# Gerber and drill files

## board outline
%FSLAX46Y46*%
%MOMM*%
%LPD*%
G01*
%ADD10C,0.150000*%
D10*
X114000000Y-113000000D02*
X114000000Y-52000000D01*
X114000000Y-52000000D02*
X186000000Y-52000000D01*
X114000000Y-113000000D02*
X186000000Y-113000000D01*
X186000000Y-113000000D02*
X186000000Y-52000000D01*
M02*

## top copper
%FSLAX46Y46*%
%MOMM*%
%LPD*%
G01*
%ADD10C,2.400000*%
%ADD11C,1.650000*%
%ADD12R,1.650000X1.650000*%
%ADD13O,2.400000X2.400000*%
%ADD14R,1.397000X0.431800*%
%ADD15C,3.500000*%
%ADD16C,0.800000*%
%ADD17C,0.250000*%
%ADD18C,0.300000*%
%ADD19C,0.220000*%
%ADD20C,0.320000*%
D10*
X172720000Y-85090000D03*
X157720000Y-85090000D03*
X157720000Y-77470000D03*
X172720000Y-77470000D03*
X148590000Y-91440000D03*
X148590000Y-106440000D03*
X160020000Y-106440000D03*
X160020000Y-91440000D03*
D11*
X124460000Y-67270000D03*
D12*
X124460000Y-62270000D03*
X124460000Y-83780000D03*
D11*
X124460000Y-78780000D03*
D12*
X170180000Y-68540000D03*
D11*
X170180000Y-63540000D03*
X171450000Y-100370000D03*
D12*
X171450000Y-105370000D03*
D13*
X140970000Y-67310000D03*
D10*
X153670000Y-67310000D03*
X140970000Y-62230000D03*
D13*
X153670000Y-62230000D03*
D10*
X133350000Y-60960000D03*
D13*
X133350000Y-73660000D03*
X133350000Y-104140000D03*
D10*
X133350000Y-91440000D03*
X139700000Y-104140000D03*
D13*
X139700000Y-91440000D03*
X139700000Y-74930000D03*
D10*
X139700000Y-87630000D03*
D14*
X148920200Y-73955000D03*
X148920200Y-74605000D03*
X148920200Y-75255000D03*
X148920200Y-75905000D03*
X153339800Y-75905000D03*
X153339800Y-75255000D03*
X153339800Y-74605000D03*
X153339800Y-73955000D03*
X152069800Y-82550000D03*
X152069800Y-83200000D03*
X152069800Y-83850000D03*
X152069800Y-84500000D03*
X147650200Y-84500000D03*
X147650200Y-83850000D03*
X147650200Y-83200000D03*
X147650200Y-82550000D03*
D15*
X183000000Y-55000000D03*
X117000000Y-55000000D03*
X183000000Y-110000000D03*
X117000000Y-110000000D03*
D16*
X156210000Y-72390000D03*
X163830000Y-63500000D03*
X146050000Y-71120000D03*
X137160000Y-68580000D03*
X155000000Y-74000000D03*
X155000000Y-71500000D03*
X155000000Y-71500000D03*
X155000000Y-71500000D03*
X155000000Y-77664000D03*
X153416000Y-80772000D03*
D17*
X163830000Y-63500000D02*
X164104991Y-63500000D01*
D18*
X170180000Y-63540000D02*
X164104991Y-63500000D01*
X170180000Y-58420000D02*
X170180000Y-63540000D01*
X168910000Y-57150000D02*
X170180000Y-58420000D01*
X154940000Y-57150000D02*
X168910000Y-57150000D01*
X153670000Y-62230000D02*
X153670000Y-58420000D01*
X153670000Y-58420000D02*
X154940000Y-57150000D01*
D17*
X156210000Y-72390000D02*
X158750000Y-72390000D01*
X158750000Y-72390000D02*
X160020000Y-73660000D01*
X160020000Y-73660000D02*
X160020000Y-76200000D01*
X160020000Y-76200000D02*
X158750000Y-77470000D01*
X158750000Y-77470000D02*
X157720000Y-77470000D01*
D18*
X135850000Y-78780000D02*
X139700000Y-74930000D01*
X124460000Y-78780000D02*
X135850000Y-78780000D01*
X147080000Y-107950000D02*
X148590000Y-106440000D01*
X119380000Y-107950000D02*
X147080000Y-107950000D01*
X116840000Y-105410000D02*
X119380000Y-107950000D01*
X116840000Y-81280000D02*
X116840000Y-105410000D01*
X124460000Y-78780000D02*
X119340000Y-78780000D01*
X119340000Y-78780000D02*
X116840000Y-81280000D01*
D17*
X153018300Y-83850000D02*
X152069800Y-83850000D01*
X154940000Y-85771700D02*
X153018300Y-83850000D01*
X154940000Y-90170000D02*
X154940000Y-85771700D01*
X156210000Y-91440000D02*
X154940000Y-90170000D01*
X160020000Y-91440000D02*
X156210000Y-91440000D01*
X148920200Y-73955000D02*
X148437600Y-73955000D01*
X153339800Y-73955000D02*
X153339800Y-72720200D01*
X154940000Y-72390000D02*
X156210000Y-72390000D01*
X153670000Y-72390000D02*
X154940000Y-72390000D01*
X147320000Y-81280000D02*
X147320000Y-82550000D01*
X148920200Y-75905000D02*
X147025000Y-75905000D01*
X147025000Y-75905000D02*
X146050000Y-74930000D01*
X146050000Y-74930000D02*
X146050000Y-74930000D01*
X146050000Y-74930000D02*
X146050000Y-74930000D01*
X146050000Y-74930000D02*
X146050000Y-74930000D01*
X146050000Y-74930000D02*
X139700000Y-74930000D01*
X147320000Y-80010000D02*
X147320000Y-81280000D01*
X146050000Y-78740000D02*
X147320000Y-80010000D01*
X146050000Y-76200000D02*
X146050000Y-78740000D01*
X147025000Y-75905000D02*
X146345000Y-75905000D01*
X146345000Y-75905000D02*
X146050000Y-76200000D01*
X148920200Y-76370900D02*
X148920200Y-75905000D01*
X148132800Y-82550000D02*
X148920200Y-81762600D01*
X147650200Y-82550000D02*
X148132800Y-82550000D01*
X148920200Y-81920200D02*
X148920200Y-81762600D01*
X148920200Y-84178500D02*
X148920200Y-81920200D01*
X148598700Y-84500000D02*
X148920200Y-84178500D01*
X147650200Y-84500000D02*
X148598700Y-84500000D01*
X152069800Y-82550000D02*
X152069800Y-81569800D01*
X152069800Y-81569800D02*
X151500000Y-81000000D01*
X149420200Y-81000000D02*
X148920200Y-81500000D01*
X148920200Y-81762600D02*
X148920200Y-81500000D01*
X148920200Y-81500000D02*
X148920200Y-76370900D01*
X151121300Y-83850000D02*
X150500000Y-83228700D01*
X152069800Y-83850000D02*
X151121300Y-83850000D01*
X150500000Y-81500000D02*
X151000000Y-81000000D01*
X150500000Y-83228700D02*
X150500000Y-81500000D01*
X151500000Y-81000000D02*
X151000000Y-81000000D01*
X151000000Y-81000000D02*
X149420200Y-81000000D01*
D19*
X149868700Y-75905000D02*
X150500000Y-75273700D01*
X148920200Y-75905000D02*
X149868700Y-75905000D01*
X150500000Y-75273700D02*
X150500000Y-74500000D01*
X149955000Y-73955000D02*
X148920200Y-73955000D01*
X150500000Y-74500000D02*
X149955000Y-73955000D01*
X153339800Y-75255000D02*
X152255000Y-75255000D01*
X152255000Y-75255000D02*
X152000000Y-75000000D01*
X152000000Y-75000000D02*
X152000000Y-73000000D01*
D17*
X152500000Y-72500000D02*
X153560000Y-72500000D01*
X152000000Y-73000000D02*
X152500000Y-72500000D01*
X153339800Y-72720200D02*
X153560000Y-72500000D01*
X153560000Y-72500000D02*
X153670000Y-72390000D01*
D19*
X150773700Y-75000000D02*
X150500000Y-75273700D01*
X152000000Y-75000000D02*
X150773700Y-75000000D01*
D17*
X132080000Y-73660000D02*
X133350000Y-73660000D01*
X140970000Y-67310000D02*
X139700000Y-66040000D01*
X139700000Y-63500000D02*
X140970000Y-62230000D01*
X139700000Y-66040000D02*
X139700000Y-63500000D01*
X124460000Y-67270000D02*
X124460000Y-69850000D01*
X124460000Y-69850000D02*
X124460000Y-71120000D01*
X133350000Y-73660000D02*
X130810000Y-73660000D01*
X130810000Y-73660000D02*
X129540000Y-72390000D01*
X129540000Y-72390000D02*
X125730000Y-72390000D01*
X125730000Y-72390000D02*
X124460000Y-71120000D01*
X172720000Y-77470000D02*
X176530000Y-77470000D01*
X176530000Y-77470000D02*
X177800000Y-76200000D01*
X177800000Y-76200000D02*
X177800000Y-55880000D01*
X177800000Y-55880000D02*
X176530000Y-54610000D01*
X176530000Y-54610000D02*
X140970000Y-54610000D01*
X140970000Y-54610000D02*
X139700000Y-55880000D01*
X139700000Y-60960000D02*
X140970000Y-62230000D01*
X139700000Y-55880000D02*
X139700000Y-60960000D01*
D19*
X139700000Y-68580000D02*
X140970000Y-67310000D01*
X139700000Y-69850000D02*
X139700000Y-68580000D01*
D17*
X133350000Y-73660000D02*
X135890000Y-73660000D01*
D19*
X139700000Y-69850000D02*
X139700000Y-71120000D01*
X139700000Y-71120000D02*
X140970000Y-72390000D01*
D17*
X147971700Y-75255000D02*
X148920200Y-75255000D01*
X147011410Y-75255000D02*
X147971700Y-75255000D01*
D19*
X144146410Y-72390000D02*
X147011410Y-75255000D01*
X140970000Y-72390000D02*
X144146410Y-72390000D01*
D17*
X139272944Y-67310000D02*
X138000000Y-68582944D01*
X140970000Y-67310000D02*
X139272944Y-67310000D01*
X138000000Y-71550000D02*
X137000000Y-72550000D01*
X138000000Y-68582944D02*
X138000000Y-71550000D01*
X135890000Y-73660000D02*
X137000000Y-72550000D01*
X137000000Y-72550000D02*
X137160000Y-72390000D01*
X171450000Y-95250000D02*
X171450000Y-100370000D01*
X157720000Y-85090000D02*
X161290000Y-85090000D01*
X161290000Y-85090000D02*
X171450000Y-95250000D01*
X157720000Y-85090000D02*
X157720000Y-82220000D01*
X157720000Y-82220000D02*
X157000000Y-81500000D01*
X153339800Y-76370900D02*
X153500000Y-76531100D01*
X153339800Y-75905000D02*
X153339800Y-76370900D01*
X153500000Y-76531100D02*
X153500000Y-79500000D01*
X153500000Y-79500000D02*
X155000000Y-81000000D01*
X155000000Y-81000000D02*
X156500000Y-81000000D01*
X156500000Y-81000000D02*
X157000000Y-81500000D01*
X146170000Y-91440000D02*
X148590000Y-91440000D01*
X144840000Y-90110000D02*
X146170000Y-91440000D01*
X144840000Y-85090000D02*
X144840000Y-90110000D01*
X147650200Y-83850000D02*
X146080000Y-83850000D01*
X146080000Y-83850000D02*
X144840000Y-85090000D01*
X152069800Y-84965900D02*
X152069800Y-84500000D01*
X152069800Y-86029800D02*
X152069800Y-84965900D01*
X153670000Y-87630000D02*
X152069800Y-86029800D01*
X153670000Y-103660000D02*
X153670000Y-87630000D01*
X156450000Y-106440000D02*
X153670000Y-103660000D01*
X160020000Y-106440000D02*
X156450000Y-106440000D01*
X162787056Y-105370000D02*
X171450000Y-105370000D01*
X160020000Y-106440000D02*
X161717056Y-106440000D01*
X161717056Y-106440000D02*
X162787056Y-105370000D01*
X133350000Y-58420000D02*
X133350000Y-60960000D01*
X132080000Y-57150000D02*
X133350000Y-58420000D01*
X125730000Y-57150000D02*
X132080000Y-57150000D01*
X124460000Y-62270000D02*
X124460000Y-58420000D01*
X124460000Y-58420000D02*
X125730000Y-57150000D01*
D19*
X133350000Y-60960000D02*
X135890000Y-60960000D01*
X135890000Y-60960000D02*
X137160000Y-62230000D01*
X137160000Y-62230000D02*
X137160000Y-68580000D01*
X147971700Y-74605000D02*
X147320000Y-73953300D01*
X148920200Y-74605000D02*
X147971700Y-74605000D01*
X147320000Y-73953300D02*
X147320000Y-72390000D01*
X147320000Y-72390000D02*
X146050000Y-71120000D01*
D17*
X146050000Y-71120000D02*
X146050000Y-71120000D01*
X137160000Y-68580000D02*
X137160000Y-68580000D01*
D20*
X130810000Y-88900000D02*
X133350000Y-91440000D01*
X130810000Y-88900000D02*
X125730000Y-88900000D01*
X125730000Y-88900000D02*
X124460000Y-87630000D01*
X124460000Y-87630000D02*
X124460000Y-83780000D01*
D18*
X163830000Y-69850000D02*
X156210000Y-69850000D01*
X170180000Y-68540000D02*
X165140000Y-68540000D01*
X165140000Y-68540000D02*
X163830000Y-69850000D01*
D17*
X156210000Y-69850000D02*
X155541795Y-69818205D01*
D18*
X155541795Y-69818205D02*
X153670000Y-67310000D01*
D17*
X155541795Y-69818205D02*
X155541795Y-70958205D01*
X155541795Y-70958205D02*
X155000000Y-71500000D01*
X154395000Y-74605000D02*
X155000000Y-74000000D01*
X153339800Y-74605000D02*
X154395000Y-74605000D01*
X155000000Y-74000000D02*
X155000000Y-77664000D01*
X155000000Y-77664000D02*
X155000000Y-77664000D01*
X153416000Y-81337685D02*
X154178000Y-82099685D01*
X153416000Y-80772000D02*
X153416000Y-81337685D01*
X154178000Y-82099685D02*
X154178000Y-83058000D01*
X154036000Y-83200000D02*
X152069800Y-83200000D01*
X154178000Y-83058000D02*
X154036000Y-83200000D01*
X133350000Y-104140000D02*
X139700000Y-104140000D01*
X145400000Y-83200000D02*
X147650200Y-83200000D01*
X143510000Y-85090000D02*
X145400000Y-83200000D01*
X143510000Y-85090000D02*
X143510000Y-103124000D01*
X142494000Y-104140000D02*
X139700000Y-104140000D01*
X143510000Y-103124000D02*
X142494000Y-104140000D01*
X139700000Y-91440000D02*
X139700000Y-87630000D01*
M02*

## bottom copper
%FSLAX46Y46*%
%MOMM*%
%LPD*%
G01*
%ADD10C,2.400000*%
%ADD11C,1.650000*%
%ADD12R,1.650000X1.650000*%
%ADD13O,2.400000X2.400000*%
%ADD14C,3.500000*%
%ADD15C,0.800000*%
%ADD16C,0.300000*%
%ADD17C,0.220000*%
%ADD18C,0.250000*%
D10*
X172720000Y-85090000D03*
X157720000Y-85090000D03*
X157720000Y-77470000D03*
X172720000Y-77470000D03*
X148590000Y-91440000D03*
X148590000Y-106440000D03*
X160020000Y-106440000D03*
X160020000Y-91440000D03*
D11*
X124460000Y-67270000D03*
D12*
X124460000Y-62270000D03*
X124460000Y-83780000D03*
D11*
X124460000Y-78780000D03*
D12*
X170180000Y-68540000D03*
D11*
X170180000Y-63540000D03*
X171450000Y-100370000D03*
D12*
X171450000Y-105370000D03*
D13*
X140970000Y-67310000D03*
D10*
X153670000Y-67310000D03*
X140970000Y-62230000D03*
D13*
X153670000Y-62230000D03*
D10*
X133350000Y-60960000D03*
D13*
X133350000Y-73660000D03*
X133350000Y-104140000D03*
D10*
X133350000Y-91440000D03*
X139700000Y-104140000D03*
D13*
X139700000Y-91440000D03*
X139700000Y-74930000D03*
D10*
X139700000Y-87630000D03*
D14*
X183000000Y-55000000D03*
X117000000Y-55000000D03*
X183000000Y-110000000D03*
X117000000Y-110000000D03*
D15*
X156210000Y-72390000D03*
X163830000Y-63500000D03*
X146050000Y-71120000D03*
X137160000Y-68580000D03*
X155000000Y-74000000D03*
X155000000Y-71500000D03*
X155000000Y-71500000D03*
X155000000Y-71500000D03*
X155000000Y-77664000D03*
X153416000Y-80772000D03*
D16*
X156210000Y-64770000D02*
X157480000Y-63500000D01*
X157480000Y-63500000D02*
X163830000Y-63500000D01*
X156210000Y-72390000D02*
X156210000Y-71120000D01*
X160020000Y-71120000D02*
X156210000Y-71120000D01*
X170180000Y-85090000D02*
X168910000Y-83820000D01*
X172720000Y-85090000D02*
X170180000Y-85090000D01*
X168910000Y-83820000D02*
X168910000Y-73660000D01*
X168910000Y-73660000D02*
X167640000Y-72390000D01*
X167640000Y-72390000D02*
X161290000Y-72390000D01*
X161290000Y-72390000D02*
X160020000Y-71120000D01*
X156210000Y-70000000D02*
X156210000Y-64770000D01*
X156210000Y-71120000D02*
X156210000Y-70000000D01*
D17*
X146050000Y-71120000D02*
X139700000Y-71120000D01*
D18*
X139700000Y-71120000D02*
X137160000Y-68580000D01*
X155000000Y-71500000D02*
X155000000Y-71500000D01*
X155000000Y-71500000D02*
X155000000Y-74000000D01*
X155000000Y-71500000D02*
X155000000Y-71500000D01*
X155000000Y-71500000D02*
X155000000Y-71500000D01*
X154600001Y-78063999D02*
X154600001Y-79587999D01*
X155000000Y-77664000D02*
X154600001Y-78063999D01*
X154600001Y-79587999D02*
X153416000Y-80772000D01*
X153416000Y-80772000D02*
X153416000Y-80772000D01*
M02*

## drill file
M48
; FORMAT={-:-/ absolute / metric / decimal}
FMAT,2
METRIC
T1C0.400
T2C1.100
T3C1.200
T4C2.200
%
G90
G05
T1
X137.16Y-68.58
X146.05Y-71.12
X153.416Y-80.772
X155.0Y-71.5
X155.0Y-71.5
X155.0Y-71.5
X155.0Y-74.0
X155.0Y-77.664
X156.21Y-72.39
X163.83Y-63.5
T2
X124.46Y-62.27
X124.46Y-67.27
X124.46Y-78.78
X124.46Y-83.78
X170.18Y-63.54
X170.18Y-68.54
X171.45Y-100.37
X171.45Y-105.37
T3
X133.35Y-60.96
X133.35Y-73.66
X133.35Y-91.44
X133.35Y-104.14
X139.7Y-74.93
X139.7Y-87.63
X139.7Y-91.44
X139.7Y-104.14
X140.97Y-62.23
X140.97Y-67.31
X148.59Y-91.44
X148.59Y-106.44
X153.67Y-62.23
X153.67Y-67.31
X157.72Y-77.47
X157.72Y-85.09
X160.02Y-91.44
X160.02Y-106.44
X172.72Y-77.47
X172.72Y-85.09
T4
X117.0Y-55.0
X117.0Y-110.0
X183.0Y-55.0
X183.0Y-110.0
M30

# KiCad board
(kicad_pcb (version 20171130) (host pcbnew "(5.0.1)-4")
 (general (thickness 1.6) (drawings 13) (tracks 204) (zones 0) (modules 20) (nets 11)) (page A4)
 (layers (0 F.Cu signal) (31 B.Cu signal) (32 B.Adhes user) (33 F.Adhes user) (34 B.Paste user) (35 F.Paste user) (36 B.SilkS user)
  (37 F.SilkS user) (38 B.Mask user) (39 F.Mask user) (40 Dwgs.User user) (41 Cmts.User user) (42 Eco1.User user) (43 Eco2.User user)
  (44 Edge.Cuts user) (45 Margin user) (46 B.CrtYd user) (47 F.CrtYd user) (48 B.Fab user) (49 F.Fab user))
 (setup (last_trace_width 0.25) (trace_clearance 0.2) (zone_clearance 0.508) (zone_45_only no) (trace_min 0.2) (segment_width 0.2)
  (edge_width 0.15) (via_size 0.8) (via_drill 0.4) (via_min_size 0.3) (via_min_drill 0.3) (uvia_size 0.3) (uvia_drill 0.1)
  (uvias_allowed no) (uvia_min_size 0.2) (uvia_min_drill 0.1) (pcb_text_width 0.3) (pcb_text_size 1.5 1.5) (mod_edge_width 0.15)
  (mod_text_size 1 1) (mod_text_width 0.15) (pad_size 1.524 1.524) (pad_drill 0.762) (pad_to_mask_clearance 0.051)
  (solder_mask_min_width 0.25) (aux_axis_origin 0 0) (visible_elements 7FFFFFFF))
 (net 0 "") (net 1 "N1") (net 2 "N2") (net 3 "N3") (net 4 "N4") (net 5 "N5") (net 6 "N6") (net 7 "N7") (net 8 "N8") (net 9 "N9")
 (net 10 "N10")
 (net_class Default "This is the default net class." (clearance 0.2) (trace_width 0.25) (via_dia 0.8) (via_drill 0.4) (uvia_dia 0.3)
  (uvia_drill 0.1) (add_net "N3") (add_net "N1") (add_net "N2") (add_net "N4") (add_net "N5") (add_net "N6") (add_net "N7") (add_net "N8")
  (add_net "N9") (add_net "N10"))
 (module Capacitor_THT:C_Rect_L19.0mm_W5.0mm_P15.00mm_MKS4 (layer F.Cu) (at 172.72 85.09 180)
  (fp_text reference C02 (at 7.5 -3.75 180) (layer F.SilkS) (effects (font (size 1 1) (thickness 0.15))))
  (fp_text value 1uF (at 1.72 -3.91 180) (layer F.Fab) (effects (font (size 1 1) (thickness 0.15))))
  (pad 1 thru_hole circle (at 0 0 180) (size 2.4 2.4) (drill 1.2) (layers *.Cu *.Mask) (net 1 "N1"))
  (pad 2 thru_hole circle (at 15 0 180) (size 2.4 2.4) (drill 1.2) (layers *.Cu *.Mask) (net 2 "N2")))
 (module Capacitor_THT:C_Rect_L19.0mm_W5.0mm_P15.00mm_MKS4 (layer F.Cu) (at 172.72 77.47 180)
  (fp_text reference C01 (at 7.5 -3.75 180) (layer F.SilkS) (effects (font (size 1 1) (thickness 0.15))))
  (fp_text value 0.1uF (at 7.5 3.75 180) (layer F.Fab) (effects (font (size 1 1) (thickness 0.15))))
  (pad 2 thru_hole circle (at 15 0 180) (size 2.4 2.4) (drill 1.2) (layers *.Cu *.Mask) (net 1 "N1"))
  (pad 1 thru_hole circle (at 0 0 180) (size 2.4 2.4) (drill 1.2) (layers *.Cu *.Mask) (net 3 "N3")))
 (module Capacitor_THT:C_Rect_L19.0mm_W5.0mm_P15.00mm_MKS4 (layer F.Cu) (at 148.59 91.44 270)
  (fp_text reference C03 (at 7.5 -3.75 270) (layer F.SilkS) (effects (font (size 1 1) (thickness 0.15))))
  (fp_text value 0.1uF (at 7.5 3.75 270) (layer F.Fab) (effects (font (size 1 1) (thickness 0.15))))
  (pad 1 thru_hole circle (at 0 0 270) (size 2.4 2.4) (drill 1.2) (layers *.Cu *.Mask) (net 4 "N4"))
  (pad 2 thru_hole circle (at 15 0 270) (size 2.4 2.4) (drill 1.2) (layers *.Cu *.Mask) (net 1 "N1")))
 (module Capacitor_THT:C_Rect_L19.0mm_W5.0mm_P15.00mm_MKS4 (layer F.Cu) (at 160.02 91.44 270)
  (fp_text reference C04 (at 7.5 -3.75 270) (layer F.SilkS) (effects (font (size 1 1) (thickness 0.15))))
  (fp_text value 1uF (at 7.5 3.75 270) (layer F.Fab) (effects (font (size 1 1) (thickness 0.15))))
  (pad 2 thru_hole circle (at 15 0 270) (size 2.4 2.4) (drill 1.2) (layers *.Cu *.Mask) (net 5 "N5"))
  (pad 1 thru_hole circle (at 0 0 270) (size 2.4 2.4) (drill 1.2) (layers *.Cu *.Mask) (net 1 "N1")))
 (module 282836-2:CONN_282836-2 (layer F.Cu) (at 124.46 64.77 270)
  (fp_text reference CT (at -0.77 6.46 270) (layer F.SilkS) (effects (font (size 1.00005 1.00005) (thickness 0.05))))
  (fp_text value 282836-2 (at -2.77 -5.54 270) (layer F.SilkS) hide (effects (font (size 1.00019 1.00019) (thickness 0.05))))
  (pad 2 thru_hole circle (at 2.5 0 270) (size 1.65 1.65) (drill 1.1) (layers *.Cu *.Mask) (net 3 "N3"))
  (pad 1 thru_hole rect (at -2.5 0 270) (size 1.65 1.65) (drill 1.1) (layers *.Cu *.Mask) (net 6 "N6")))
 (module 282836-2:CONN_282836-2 (layer F.Cu) (at 124.46 81.28 90)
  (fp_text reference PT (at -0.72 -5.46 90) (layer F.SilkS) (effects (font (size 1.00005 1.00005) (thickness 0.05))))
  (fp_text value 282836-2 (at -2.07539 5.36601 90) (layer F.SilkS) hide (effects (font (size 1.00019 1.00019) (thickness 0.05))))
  (pad 1 thru_hole rect (at -2.5 0 90) (size 1.65 1.65) (drill 1.1) (layers *.Cu *.Mask) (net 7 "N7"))
  (pad 2 thru_hole circle (at 2.5 0 90) (size 1.65 1.65) (drill 1.1) (layers *.Cu *.Mask) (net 1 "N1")))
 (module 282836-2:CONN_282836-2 (layer F.Cu) (at 170.18 66.04 90)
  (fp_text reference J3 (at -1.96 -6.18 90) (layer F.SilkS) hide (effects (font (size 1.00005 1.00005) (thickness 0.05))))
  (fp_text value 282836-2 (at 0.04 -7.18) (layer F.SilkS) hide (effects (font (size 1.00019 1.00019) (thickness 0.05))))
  (pad 1 thru_hole rect (at -2.5 0 90) (size 1.65 1.65) (drill 1.1) (layers *.Cu *.Mask) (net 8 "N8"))
  (pad 2 thru_hole circle (at 2.5 0 90) (size 1.65 1.65) (drill 1.1) (layers *.Cu *.Mask) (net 1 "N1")))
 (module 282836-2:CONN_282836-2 (layer F.Cu) (at 171.45 102.87 90)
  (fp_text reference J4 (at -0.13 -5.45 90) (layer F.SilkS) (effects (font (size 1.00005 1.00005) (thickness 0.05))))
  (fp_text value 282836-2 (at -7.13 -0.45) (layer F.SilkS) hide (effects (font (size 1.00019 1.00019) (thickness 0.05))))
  (pad 2 thru_hole circle (at 2.5 0 90) (size 1.65 1.65) (drill 1.1) (layers *.Cu *.Mask) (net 2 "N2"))
  (pad 1 thru_hole rect (at -2.5 0 90) (size 1.65 1.65) (drill 1.1) (layers *.Cu *.Mask) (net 5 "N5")))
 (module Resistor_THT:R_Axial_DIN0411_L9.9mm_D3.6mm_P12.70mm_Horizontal (layer F.Cu) (at 153.67 67.31 180)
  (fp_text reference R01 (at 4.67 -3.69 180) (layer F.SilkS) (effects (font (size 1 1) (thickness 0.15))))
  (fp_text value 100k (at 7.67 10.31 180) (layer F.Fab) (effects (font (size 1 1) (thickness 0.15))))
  (pad 2 thru_hole oval (at 12.7 0 180) (size 2.4 2.4) (drill 1.2) (layers *.Cu *.Mask) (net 3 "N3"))
  (pad 1 thru_hole circle (at 0 0 180) (size 2.4 2.4) (drill 1.2) (layers *.Cu *.Mask) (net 8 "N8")))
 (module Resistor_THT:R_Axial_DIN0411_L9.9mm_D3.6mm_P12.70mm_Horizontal (layer F.Cu) (at 140.97 62.23)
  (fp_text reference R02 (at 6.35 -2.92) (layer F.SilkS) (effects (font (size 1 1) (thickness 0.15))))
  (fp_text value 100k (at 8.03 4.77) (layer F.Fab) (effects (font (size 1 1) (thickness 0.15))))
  (pad 1 thru_hole circle (at 0 0) (size 2.4 2.4) (drill 1.2) (layers *.Cu *.Mask) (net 3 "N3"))
  (pad 2 thru_hole oval (at 12.7 0) (size 2.4 2.4) (drill 1.2) (layers *.Cu *.Mask) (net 1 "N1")))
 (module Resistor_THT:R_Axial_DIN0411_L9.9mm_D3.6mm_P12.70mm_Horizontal (layer F.Cu) (at 133.35 60.96 270)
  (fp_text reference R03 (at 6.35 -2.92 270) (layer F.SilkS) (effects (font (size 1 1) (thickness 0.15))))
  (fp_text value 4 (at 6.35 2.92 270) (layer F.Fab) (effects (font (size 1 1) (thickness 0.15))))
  (pad 1 thru_hole circle (at 0 0 270) (size 2.4 2.4) (drill 1.2) (layers *.Cu *.Mask) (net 6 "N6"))
  (pad 2 thru_hole oval (at 12.7 0 270) (size 2.4 2.4) (drill 1.2) (layers *.Cu *.Mask) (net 3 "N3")))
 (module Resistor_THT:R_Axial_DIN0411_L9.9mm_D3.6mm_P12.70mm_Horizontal (layer F.Cu) (at 133.35 91.44 270)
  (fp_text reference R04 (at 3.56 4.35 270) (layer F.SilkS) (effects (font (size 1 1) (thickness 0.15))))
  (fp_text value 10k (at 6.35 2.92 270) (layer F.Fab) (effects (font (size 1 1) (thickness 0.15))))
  (pad 2 thru_hole oval (at 12.7 0 270) (size 2.4 2.4) (drill 1.2) (layers *.Cu *.Mask) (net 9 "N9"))
  (pad 1 thru_hole circle (at 0 0 270) (size 2.4 2.4) (drill 1.2) (layers *.Cu *.Mask) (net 7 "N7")))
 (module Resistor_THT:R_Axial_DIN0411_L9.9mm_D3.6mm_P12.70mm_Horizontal (layer F.Cu) (at 139.7 104.14 90)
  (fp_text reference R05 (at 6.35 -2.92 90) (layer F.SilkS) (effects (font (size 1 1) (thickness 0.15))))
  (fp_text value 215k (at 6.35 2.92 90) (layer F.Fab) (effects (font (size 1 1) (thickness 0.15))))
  (pad 1 thru_hole circle (at 0 0 90) (size 2.4 2.4) (drill 1.2) (layers *.Cu *.Mask) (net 9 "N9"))
  (pad 2 thru_hole oval (at 12.7 0 90) (size 2.4 2.4) (drill 1.2) (layers *.Cu *.Mask) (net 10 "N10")))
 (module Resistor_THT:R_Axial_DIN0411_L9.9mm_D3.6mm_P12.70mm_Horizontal (layer F.Cu) (at 139.7 87.63 90)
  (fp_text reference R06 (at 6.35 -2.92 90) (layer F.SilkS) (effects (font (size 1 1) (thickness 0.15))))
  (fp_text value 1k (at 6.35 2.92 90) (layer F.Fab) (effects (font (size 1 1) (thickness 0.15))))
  (pad 2 thru_hole oval (at 12.7 0 90) (size 2.4 2.4) (drill 1.2) (layers *.Cu *.Mask) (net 1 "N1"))
  (pad 1 thru_hole circle (at 0 0 90) (size 2.4 2.4) (drill 1.2) (layers *.Cu *.Mask) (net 10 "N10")))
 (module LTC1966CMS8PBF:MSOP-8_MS (layer F.Cu) (at 151.13 74.93)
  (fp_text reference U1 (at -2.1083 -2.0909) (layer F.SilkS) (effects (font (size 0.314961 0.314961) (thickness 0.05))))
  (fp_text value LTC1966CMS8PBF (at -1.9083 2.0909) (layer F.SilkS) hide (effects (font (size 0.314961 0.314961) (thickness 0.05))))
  (pad 1 smd rect (at -2.2098 -0.975) (size 1.397 0.4318) (layers F.Cu F.Paste F.Mask) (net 1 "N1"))
  (pad 2 smd rect (at -2.2098 -0.325) (size 1.397 0.4318) (layers F.Cu F.Paste F.Mask) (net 6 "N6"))
  (pad 3 smd rect (at -2.2098 0.325) (size 1.397 0.4318) (layers F.Cu F.Paste F.Mask) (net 3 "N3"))
  (pad 4 smd rect (at -2.2098 0.975) (size 1.397 0.4318) (layers F.Cu F.Paste F.Mask) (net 1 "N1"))
  (pad 5 smd rect (at 2.2098 0.975) (size 1.397 0.4318) (layers F.Cu F.Paste F.Mask) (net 2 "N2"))
  (pad 6 smd rect (at 2.2098 0.325) (size 1.397 0.4318) (layers F.Cu F.Paste F.Mask) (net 1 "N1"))
  (pad 7 smd rect (at 2.2098 -0.325) (size 1.397 0.4318) (layers F.Cu F.Paste F.Mask) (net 8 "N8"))
  (pad 8 smd rect (at 2.2098 -0.975) (size 1.397 0.4318) (layers F.Cu F.Paste F.Mask) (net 1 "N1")))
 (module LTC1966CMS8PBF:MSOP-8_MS (layer F.Cu) (at 149.86 83.525)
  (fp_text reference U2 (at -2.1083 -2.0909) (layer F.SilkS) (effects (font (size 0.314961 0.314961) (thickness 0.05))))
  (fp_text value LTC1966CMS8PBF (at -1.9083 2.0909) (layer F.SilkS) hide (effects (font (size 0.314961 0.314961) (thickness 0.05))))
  (pad 8 smd rect (at 2.2098 -0.975) (size 1.397 0.4318) (layers F.Cu F.Paste F.Mask) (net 1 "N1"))
  (pad 7 smd rect (at 2.2098 -0.325) (size 1.397 0.4318) (layers F.Cu F.Paste F.Mask) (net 8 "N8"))
  (pad 6 smd rect (at 2.2098 0.325) (size 1.397 0.4318) (layers F.Cu F.Paste F.Mask) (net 1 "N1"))
  (pad 5 smd rect (at 2.2098 0.975) (size 1.397 0.4318) (layers F.Cu F.Paste F.Mask) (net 5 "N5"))
  (pad 4 smd rect (at -2.2098 0.975) (size 1.397 0.4318) (layers F.Cu F.Paste F.Mask) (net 1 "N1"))
  (pad 3 smd rect (at -2.2098 0.325) (size 1.397 0.4318) (layers F.Cu F.Paste F.Mask) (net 4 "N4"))
  (pad 2 smd rect (at -2.2098 -0.325) (size 1.397 0.4318) (layers F.Cu F.Paste F.Mask) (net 9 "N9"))
  (pad 1 smd rect (at -2.2098 -0.975) (size 1.397 0.4318) (layers F.Cu F.Paste F.Mask) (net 1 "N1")))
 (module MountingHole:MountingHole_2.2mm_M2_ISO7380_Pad (layer F.Cu) (at 183 55)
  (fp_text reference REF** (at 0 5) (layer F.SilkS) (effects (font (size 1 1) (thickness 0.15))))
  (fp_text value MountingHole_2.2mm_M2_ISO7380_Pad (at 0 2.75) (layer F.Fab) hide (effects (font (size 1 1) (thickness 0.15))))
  (pad 1 thru_hole circle (at 0 0) (size 3.5 3.5) (drill 2.2) (layers *.Cu *.Mask)))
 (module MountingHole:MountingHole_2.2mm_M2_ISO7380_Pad (layer F.Cu) (at 117 55)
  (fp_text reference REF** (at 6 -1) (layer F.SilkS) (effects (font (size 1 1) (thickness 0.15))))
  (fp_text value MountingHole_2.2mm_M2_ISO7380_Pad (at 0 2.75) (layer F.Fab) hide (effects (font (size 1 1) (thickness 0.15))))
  (pad 1 thru_hole circle (at 0 0) (size 3.5 3.5) (drill 2.2) (layers *.Cu *.Mask)))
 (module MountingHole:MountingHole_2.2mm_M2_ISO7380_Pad (layer F.Cu) (at 183 110)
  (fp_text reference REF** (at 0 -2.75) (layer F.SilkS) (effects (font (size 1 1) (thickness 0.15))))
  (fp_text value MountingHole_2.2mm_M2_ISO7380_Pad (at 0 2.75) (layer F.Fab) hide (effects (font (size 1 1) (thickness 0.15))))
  (pad 1 thru_hole circle (at 0 0) (size 3.5 3.5) (drill 2.2) (layers *.Cu *.Mask)))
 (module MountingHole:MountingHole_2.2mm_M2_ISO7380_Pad (layer F.Cu) (at 117 110)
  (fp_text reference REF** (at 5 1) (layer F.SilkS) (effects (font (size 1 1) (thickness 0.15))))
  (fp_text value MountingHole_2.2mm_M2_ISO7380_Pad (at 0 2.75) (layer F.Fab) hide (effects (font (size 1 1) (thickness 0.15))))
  (pad 1 thru_hole circle (at 0 0) (size 3.5 3.5) (drill 2.2) (layers *.Cu *.Mask)))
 (gr_line (start 114 113) (end 114 52) (layer Edge.Cuts) (width 0.15))
 (gr_line (start 114 52) (end 186 52) (layer Edge.Cuts) (width 0.15))
 (gr_line (start 114 113) (end 186 113) (layer Edge.Cuts) (width 0.15))
 (gr_line (start 186 113) (end 186 52) (layer Edge.Cuts) (width 0.15))
 (via (at 156.21 72.39) (size 0.8) (drill 0.4) (layers F.Cu B.Cu) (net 1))
 (via (at 163.83 63.5) (size 0.8) (drill 0.4) (layers F.Cu B.Cu) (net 1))
 (segment (start 163.83 63.5) (end 164.104991 63.5) (width 0.25) (layer F.Cu) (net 1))
 (segment (start 170.18 63.54) (end 164.104991 63.5) (width 0.3) (layer F.Cu) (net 1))
 (segment (start 170.18 58.42) (end 170.18 63.54) (width 0.3) (layer F.Cu) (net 1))
 (segment (start 168.91 57.15) (end 170.18 58.42) (width 0.3) (layer F.Cu) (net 1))
 (segment (start 154.94 57.15) (end 168.91 57.15) (width 0.3) (layer F.Cu) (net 1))
 (segment (start 153.67 62.23) (end 153.67 58.42) (width 0.3) (layer F.Cu) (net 1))
 (segment (start 153.67 58.42) (end 154.94 57.15) (width 0.3) (layer F.Cu) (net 1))
 (segment (start 156.21 64.77) (end 157.48 63.5) (width 0.3) (layer B.Cu) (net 1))
 (segment (start 157.48 63.5) (end 163.83 63.5) (width 0.3) (layer B.Cu) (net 1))
 (segment (start 156.21 72.39) (end 158.75 72.39) (width 0.25) (layer F.Cu) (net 1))
 (segment (start 158.75 72.39) (end 160.02 73.66) (width 0.25) (layer F.Cu) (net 1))
 (segment (start 160.02 73.66) (end 160.02 76.2) (width 0.25) (layer F.Cu) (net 1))
 (segment (start 160.02 76.2) (end 158.75 77.47) (width 0.25) (layer F.Cu) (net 1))
 (segment (start 158.75 77.47) (end 157.72 77.47) (width 0.25) (layer F.Cu) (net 1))
 (segment (start 156.21 72.39) (end 156.21 71.12) (width 0.3) (layer B.Cu) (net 1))
 (segment (start 160.02 71.12) (end 156.21 71.12) (width 0.3) (layer B.Cu) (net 1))
 (segment (start 170.18 85.09) (end 168.91 83.82) (width 0.3) (layer B.Cu) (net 1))
 (segment (start 172.72 85.09) (end 170.18 85.09) (width 0.3) (layer B.Cu) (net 1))
 (segment (start 168.91 83.82) (end 168.91 73.66) (width 0.3) (layer B.Cu) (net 1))
 (segment (start 168.91 73.66) (end 167.64 72.39) (width 0.3) (layer B.Cu) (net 1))
 (segment (start 167.64 72.39) (end 161.29 72.39) (width 0.3) (layer B.Cu) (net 1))
 (segment (start 161.29 72.39) (end 160.02 71.12) (width 0.3) (layer B.Cu) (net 1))
 (segment (start 135.85 78.78) (end 139.7 74.93) (width 0.3) (layer F.Cu) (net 1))
 (segment (start 124.46 78.78) (end 135.85 78.78) (width 0.3) (layer F.Cu) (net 1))
 (segment (start 147.08 107.95) (end 148.59 106.44) (width 0.3) (layer F.Cu) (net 1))
 (segment (start 119.38 107.95) (end 147.08 107.95) (width 0.3) (layer F.Cu) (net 1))
 (segment (start 116.84 105.41) (end 119.38 107.95) (width 0.3) (layer F.Cu) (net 1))
 (segment (start 116.84 81.28) (end 116.84 105.41) (width 0.3) (layer F.Cu) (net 1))
 (segment (start 124.46 78.78) (end 119.34 78.78) (width 0.3) (layer F.Cu) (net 1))
 (segment (start 119.34 78.78) (end 116.84 81.28) (width 0.3) (layer F.Cu) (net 1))
 (segment (start 153.0183 83.85) (end 152.0698 83.85) (width 0.25) (layer F.Cu) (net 1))
 (segment (start 154.94 85.7717) (end 153.0183 83.85) (width 0.25) (layer F.Cu) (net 1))
 (segment (start 154.94 90.17) (end 154.94 85.7717) (width 0.25) (layer F.Cu) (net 1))
 (segment (start 156.21 91.44) (end 154.94 90.17) (width 0.25) (layer F.Cu) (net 1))
 (segment (start 160.02 91.44) (end 156.21 91.44) (width 0.25) (layer F.Cu) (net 1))
 (segment (start 148.9202 73.955) (end 148.4376 73.955) (width 0.25) (layer F.Cu) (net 1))
 (segment (start 153.3398 73.955) (end 153.3398 72.7202) (width 0.25) (layer F.Cu) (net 1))
 (segment (start 154.94 72.39) (end 156.21 72.39) (width 0.25) (layer F.Cu) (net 1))
 (segment (start 153.67 72.39) (end 154.94 72.39) (width 0.25) (layer F.Cu) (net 1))
 (segment (start 147.32 81.28) (end 147.32 82.55) (width 0.25) (layer F.Cu) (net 1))
 (segment (start 148.9202 75.905) (end 147.025 75.905) (width 0.25) (layer F.Cu) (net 1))
 (segment (start 147.025 75.905) (end 146.05 74.93) (width 0.25) (layer F.Cu) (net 1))
 (segment (start 146.05 74.93) (end 146.05 74.93) (width 0.25) (layer F.Cu) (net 1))
 (segment (start 146.05 74.93) (end 146.05 74.93) (width 0.25) (layer F.Cu) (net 1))
 (segment (start 146.05 74.93) (end 146.05 74.93) (width 0.25) (layer F.Cu) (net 1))
 (segment (start 146.05 74.93) (end 139.7 74.93) (width 0.25) (layer F.Cu) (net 1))
 (segment (start 147.32 80.01) (end 147.32 81.28) (width 0.25) (layer F.Cu) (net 1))
 (segment (start 146.05 78.74) (end 147.32 80.01) (width 0.25) (layer F.Cu) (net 1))
 (segment (start 146.05 76.2) (end 146.05 78.74) (width 0.25) (layer F.Cu) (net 1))
 (segment (start 147.025 75.905) (end 146.345 75.905) (width 0.25) (layer F.Cu) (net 1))
 (segment (start 146.345 75.905) (end 146.05 76.2) (width 0.25) (layer F.Cu) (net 1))
 (segment (start 148.9202 76.3709) (end 148.9202 75.905) (width 0.25) (layer F.Cu) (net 1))
 (segment (start 148.1328 82.55) (end 148.9202 81.7626) (width 0.25) (layer F.Cu) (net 1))
 (segment (start 147.6502 82.55) (end 148.1328 82.55) (width 0.25) (layer F.Cu) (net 1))
 (segment (start 148.9202 81.9202) (end 148.9202 81.7626) (width 0.25) (layer F.Cu) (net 1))
 (segment (start 148.9202 84.1785) (end 148.9202 81.9202) (width 0.25) (layer F.Cu) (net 1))
 (segment (start 148.5987 84.5) (end 148.9202 84.1785) (width 0.25) (layer F.Cu) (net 1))
 (segment (start 147.6502 84.5) (end 148.5987 84.5) (width 0.25) (layer F.Cu) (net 1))
 (segment (start 152.0698 82.55) (end 152.0698 81.5698) (width 0.25) (layer F.Cu) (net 1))
 (segment (start 152.0698 81.5698) (end 151.5 81) (width 0.25) (layer F.Cu) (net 1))
 (segment (start 149.4202 81) (end 148.9202 81.5) (width 0.25) (layer F.Cu) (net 1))
 (segment (start 148.9202 81.7626) (end 148.9202 81.5) (width 0.25) (layer F.Cu) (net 1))
 (segment (start 148.9202 81.5) (end 148.9202 76.3709) (width 0.25) (layer F.Cu) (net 1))
 (segment (start 151.1213 83.85) (end 150.5 83.2287) (width 0.25) (layer F.Cu) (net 1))
 (segment (start 152.0698 83.85) (end 151.1213 83.85) (width 0.25) (layer F.Cu) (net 1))
 (segment (start 150.5 81.5) (end 151 81) (width 0.25) (layer F.Cu) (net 1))
 (segment (start 150.5 83.2287) (end 150.5 81.5) (width 0.25) (layer F.Cu) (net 1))
 (segment (start 151.5 81) (end 151 81) (width 0.25) (layer F.Cu) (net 1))
 (segment (start 151 81) (end 149.4202 81) (width 0.25) (layer F.Cu) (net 1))
 (segment (start 149.8687 75.905) (end 150.5 75.2737) (width 0.22) (layer F.Cu) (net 1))
 (segment (start 148.9202 75.905) (end 149.8687 75.905) (width 0.22) (layer F.Cu) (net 1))
 (segment (start 150.5 75.2737) (end 150.5 74.5) (width 0.22) (layer F.Cu) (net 1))
 (segment (start 149.955 73.955) (end 148.9202 73.955) (width 0.22) (layer F.Cu) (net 1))
 (segment (start 150.5 74.5) (end 149.955 73.955) (width 0.22) (layer F.Cu) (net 1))
 (segment (start 153.3398 75.255) (end 152.255 75.255) (width 0.22) (layer F.Cu) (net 1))
 (segment (start 152.255 75.255) (end 152 75) (width 0.22) (layer F.Cu) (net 1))
 (segment (start 152 75) (end 152 73) (width 0.22) (layer F.Cu) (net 1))
 (segment (start 152.5 72.5) (end 153.56 72.5) (width 0.25) (layer F.Cu) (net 1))
 (segment (start 152 73) (end 152.5 72.5) (width 0.25) (layer F.Cu) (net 1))
 (segment (start 153.3398 72.7202) (end 153.56 72.5) (width 0.25) (layer F.Cu) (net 1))
 (segment (start 153.56 72.5) (end 153.67 72.39) (width 0.25) (layer F.Cu) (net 1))
 (segment (start 156.21 70) (end 156.21 64.77) (width 0.3) (layer B.Cu) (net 1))
 (segment (start 156.21 71.12) (end 156.21 70) (width 0.3) (layer B.Cu) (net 1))
 (segment (start 150.7737 75) (end 150.5 75.2737) (width 0.22) (layer F.Cu) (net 1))
 (segment (start 152 75) (end 150.7737 75) (width 0.22) (layer F.Cu) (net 1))
 (segment (start 132.08 73.66) (end 133.35 73.66) (width 0.25) (layer F.Cu) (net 3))
 (segment (start 140.97 67.31) (end 139.7 66.04) (width 0.25) (layer F.Cu) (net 3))
 (segment (start 139.7 63.5) (end 140.97 62.23) (width 0.25) (layer F.Cu) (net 3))
 (segment (start 139.7 66.04) (end 139.7 63.5) (width 0.25) (layer F.Cu) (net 3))
 (segment (start 124.46 67.27) (end 124.46 69.85) (width 0.25) (layer F.Cu) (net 3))
 (segment (start 124.46 69.85) (end 124.46 71.12) (width 0.25) (layer F.Cu) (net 3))
 (segment (start 133.35 73.66) (end 130.81 73.66) (width 0.25) (layer F.Cu) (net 3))
 (segment (start 130.81 73.66) (end 129.54 72.39) (width 0.25) (layer F.Cu) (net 3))
 (segment (start 129.54 72.39) (end 125.73 72.39) (width 0.25) (layer F.Cu) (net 3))
 (segment (start 125.73 72.39) (end 124.46 71.12) (width 0.25) (layer F.Cu) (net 3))
 (segment (start 172.72 77.47) (end 176.53 77.47) (width 0.25) (layer F.Cu) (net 3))
 (segment (start 176.53 77.47) (end 177.8 76.2) (width 0.25) (layer F.Cu) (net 3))
 (segment (start 177.8 76.2) (end 177.8 55.88) (width 0.25) (layer F.Cu) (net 3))
 (segment (start 177.8 55.88) (end 176.53 54.61) (width 0.25) (layer F.Cu) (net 3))
 (segment (start 176.53 54.61) (end 140.97 54.61) (width 0.25) (layer F.Cu) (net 3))
 (segment (start 140.97 54.61) (end 139.7 55.88) (width 0.25) (layer F.Cu) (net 3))
 (segment (start 139.7 60.96) (end 140.97 62.23) (width 0.25) (layer F.Cu) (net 3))
 (segment (start 139.7 55.88) (end 139.7 60.96) (width 0.25) (layer F.Cu) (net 3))
 (segment (start 139.7 68.58) (end 140.97 67.31) (width 0.22) (layer F.Cu) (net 3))
 (segment (start 139.7 69.85) (end 139.7 68.58) (width 0.22) (layer F.Cu) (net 3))
 (segment (start 133.35 73.66) (end 135.89 73.66) (width 0.25) (layer F.Cu) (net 3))
 (segment (start 139.7 69.85) (end 139.7 71.12) (width 0.22) (layer F.Cu) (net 3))
 (segment (start 139.7 71.12) (end 140.97 72.39) (width 0.22) (layer F.Cu) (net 3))
 (segment (start 147.9717 75.255) (end 148.9202 75.255) (width 0.25) (layer F.Cu) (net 3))
 (segment (start 147.01141 75.255) (end 147.9717 75.255) (width 0.25) (layer F.Cu) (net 3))
 (segment (start 144.14641 72.39) (end 147.01141 75.255) (width 0.22) (layer F.Cu) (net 3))
 (segment (start 140.97 72.39) (end 144.14641 72.39) (width 0.22) (layer F.Cu) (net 3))
 (segment (start 139.272944 67.31) (end 138 68.582944) (width 0.25) (layer F.Cu) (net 3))
 (segment (start 140.97 67.31) (end 139.272944 67.31) (width 0.25) (layer F.Cu) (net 3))
 (segment (start 138 71.55) (end 137 72.55) (width 0.25) (layer F.Cu) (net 3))
 (segment (start 138 68.582944) (end 138 71.55) (width 0.25) (layer F.Cu) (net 3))
 (segment (start 135.89 73.66) (end 137 72.55) (width 0.25) (layer F.Cu) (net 3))
 (segment (start 137 72.55) (end 137.16 72.39) (width 0.25) (layer F.Cu) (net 3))
 (segment (start 171.45 95.25) (end 171.45 100.37) (width 0.25) (layer F.Cu) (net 2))
 (segment (start 157.72 85.09) (end 161.29 85.09) (width 0.25) (layer F.Cu) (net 2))
 (segment (start 161.29 85.09) (end 171.45 95.25) (width 0.25) (layer F.Cu) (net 2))
 (segment (start 157.72 85.09) (end 157.72 82.22) (width 0.25) (layer F.Cu) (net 2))
 (segment (start 157.72 82.22) (end 157 81.5) (width 0.25) (layer F.Cu) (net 2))
 (segment (start 153.3398 76.3709) (end 153.5 76.5311) (width 0.25) (layer F.Cu) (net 2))
 (segment (start 153.3398 75.905) (end 153.3398 76.3709) (width 0.25) (layer F.Cu) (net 2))
 (segment (start 153.5 76.5311) (end 153.5 79.5) (width 0.25) (layer F.Cu) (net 2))
 (segment (start 153.5 79.5) (end 155 81) (width 0.25) (layer F.Cu) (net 2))
 (segment (start 155 81) (end 156.5 81) (width 0.25) (layer F.Cu) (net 2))
 (segment (start 156.5 81) (end 157 81.5) (width 0.25) (layer F.Cu) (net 2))
 (segment (start 146.17 91.44) (end 148.59 91.44) (width 0.25) (layer F.Cu) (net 4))
 (segment (start 144.84 90.11) (end 146.17 91.44) (width 0.25) (layer F.Cu) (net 4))
 (segment (start 144.84 85.09) (end 144.84 90.11) (width 0.25) (layer F.Cu) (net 4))
 (segment (start 147.6502 83.85) (end 146.08 83.85) (width 0.25) (layer F.Cu) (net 4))
 (segment (start 146.08 83.85) (end 144.84 85.09) (width 0.25) (layer F.Cu) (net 4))
 (segment (start 152.0698 84.9659) (end 152.0698 84.5) (width 0.25) (layer F.Cu) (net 5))
 (segment (start 152.0698 86.0298) (end 152.0698 84.9659) (width 0.25) (layer F.Cu) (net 5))
 (segment (start 153.67 87.63) (end 152.0698 86.0298) (width 0.25) (layer F.Cu) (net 5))
 (segment (start 153.67 103.66) (end 153.67 87.63) (width 0.25) (layer F.Cu) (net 5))
 (segment (start 156.45 106.44) (end 153.67 103.66) (width 0.25) (layer F.Cu) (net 5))
 (segment (start 160.02 106.44) (end 156.45 106.44) (width 0.25) (layer F.Cu) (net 5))
 (segment (start 162.787056 105.37) (end 171.45 105.37) (width 0.25) (layer F.Cu) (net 5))
 (segment (start 160.02 106.44) (end 161.717056 106.44) (width 0.25) (layer F.Cu) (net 5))
 (segment (start 161.717056 106.44) (end 162.787056 105.37) (width 0.25) (layer F.Cu) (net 5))
 (segment (start 133.35 58.42) (end 133.35 60.96) (width 0.25) (layer F.Cu) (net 6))
 (segment (start 132.08 57.15) (end 133.35 58.42) (width 0.25) (layer F.Cu) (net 6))
 (segment (start 125.73 57.15) (end 132.08 57.15) (width 0.25) (layer F.Cu) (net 6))
 (segment (start 124.46 62.27) (end 124.46 58.42) (width 0.25) (layer F.Cu) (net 6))
 (segment (start 124.46 58.42) (end 125.73 57.15) (width 0.25) (layer F.Cu) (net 6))
 (segment (start 133.35 60.96) (end 135.89 60.96) (width 0.22) (layer F.Cu) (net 6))
 (segment (start 135.89 60.96) (end 137.16 62.23) (width 0.22) (layer F.Cu) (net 6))
 (segment (start 137.16 62.23) (end 137.16 68.58) (width 0.22) (layer F.Cu) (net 6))
 (segment (start 147.9717 74.605) (end 147.32 73.9533) (width 0.22) (layer F.Cu) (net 6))
 (segment (start 148.9202 74.605) (end 147.9717 74.605) (width 0.22) (layer F.Cu) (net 6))
 (segment (start 147.32 73.9533) (end 147.32 72.39) (width 0.22) (layer F.Cu) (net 6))
 (segment (start 147.32 72.39) (end 146.05 71.12) (width 0.22) (layer F.Cu) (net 6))
 (segment (start 146.05 71.12) (end 146.05 71.12) (width 0.25) (layer F.Cu) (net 6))
 (via (at 146.05 71.12) (size 0.8) (drill 0.4) (layers F.Cu B.Cu) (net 6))
 (segment (start 137.16 68.58) (end 137.16 68.58) (width 0.25) (layer F.Cu) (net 6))
 (via (at 137.16 68.58) (size 0.8) (drill 0.4) (layers F.Cu B.Cu) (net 6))
 (segment (start 146.05 71.12) (end 139.7 71.12) (width 0.22) (layer B.Cu) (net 6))
 (segment (start 139.7 71.12) (end 137.16 68.58) (width 0.25) (layer B.Cu) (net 6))
 (segment (start 130.81 88.9) (end 133.35 91.44) (width 0.32) (layer F.Cu) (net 7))
 (segment (start 130.81 88.9) (end 125.73 88.9) (width 0.32) (layer F.Cu) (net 7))
 (segment (start 125.73 88.9) (end 124.46 87.63) (width 0.32) (layer F.Cu) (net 7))
 (segment (start 124.46 87.63) (end 124.46 83.78) (width 0.32) (layer F.Cu) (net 7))
 (via (at 155 74) (size 0.8) (drill 0.4) (layers F.Cu B.Cu) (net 8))
 (segment (start 155 71.5) (end 155 71.5) (width 0.25) (layer B.Cu) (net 8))
 (segment (start 155 71.5) (end 155 74) (width 0.25) (layer B.Cu) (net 8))
 (via (at 155 71.5) (size 0.8) (drill 0.4) (layers F.Cu B.Cu) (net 8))
 (segment (start 163.83 69.85) (end 156.21 69.85) (width 0.3) (layer F.Cu) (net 8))
 (segment (start 170.18 68.54) (end 165.14 68.54) (width 0.3) (layer F.Cu) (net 8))
 (segment (start 165.14 68.54) (end 163.83 69.85) (width 0.3) (layer F.Cu) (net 8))
 (segment (start 156.21 69.85) (end 155.541795 69.818205) (width 0.25) (layer F.Cu) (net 8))
 (segment (start 155.541795 69.818205) (end 153.67 67.31) (width 0.3) (layer F.Cu) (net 8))
 (segment (start 155.541795 69.818205) (end 155.541795 70.958205) (width 0.25) (layer F.Cu) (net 8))
 (segment (start 155.541795 70.958205) (end 155 71.5) (width 0.25) (layer F.Cu) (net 8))
 (segment (start 155 71.5) (end 155 71.5) (width 0.25) (layer B.Cu) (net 8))
 (via (at 155 71.5) (size 0.8) (drill 0.4) (layers F.Cu B.Cu) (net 8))
 (segment (start 155 71.5) (end 155 71.5) (width 0.25) (layer B.Cu) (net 8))
 (via (at 155 71.5) (size 0.8) (drill 0.4) (layers F.Cu B.Cu) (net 8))
 (segment (start 154.395 74.605) (end 155 74) (width 0.25) (layer F.Cu) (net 8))
 (segment (start 153.3398 74.605) (end 154.395 74.605) (width 0.25) (layer F.Cu) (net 8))
 (segment (start 155 74) (end 155 77.664) (width 0.25) (layer F.Cu) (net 8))
 (segment (start 155 77.664) (end 155 77.664) (width 0.25) (layer F.Cu) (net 8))
 (via (at 155 77.664) (size 0.8) (drill 0.4) (layers F.Cu B.Cu) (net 8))
 (segment (start 154.600001 78.063999) (end 154.600001 79.587999) (width 0.25) (layer B.Cu) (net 8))
 (segment (start 155 77.664) (end 154.600001 78.063999) (width 0.25) (layer B.Cu) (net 8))
 (segment (start 154.600001 79.587999) (end 153.416 80.772) (width 0.25) (layer B.Cu) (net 8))
 (segment (start 153.416 80.772) (end 153.416 80.772) (width 0.25) (layer B.Cu) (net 8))
 (via (at 153.416 80.772) (size 0.8) (drill 0.4) (layers F.Cu B.Cu) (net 8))
 (segment (start 153.416 81.337685) (end 154.178 82.099685) (width 0.25) (layer F.Cu) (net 8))
 (segment (start 153.416 80.772) (end 153.416 81.337685) (width 0.25) (layer F.Cu) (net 8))
 (segment (start 154.178 82.099685) (end 154.178 83.058) (width 0.25) (layer F.Cu) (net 8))
 (segment (start 154.036 83.2) (end 152.0698 83.2) (width 0.25) (layer F.Cu) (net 8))
 (segment (start 154.178 83.058) (end 154.036 83.2) (width 0.25) (layer F.Cu) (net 8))
 (segment (start 133.35 104.14) (end 139.7 104.14) (width 0.25) (layer F.Cu) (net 9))
 (segment (start 145.4 83.2) (end 147.6502 83.2) (width 0.25) (layer F.Cu) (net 9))
 (segment (start 143.51 85.09) (end 145.4 83.2) (width 0.25) (layer F.Cu) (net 9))
 (segment (start 143.51 85.09) (end 143.51 103.124) (width 0.25) (layer F.Cu) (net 9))
 (segment (start 142.494 104.14) (end 139.7 104.14) (width 0.25) (layer F.Cu) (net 9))
 (segment (start 143.51 103.124) (end 142.494 104.14) (width 0.25) (layer F.Cu) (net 9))
 (segment (start 139.7 91.44) (end 139.7 87.63) (width 0.25) (layer F.Cu) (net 10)))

